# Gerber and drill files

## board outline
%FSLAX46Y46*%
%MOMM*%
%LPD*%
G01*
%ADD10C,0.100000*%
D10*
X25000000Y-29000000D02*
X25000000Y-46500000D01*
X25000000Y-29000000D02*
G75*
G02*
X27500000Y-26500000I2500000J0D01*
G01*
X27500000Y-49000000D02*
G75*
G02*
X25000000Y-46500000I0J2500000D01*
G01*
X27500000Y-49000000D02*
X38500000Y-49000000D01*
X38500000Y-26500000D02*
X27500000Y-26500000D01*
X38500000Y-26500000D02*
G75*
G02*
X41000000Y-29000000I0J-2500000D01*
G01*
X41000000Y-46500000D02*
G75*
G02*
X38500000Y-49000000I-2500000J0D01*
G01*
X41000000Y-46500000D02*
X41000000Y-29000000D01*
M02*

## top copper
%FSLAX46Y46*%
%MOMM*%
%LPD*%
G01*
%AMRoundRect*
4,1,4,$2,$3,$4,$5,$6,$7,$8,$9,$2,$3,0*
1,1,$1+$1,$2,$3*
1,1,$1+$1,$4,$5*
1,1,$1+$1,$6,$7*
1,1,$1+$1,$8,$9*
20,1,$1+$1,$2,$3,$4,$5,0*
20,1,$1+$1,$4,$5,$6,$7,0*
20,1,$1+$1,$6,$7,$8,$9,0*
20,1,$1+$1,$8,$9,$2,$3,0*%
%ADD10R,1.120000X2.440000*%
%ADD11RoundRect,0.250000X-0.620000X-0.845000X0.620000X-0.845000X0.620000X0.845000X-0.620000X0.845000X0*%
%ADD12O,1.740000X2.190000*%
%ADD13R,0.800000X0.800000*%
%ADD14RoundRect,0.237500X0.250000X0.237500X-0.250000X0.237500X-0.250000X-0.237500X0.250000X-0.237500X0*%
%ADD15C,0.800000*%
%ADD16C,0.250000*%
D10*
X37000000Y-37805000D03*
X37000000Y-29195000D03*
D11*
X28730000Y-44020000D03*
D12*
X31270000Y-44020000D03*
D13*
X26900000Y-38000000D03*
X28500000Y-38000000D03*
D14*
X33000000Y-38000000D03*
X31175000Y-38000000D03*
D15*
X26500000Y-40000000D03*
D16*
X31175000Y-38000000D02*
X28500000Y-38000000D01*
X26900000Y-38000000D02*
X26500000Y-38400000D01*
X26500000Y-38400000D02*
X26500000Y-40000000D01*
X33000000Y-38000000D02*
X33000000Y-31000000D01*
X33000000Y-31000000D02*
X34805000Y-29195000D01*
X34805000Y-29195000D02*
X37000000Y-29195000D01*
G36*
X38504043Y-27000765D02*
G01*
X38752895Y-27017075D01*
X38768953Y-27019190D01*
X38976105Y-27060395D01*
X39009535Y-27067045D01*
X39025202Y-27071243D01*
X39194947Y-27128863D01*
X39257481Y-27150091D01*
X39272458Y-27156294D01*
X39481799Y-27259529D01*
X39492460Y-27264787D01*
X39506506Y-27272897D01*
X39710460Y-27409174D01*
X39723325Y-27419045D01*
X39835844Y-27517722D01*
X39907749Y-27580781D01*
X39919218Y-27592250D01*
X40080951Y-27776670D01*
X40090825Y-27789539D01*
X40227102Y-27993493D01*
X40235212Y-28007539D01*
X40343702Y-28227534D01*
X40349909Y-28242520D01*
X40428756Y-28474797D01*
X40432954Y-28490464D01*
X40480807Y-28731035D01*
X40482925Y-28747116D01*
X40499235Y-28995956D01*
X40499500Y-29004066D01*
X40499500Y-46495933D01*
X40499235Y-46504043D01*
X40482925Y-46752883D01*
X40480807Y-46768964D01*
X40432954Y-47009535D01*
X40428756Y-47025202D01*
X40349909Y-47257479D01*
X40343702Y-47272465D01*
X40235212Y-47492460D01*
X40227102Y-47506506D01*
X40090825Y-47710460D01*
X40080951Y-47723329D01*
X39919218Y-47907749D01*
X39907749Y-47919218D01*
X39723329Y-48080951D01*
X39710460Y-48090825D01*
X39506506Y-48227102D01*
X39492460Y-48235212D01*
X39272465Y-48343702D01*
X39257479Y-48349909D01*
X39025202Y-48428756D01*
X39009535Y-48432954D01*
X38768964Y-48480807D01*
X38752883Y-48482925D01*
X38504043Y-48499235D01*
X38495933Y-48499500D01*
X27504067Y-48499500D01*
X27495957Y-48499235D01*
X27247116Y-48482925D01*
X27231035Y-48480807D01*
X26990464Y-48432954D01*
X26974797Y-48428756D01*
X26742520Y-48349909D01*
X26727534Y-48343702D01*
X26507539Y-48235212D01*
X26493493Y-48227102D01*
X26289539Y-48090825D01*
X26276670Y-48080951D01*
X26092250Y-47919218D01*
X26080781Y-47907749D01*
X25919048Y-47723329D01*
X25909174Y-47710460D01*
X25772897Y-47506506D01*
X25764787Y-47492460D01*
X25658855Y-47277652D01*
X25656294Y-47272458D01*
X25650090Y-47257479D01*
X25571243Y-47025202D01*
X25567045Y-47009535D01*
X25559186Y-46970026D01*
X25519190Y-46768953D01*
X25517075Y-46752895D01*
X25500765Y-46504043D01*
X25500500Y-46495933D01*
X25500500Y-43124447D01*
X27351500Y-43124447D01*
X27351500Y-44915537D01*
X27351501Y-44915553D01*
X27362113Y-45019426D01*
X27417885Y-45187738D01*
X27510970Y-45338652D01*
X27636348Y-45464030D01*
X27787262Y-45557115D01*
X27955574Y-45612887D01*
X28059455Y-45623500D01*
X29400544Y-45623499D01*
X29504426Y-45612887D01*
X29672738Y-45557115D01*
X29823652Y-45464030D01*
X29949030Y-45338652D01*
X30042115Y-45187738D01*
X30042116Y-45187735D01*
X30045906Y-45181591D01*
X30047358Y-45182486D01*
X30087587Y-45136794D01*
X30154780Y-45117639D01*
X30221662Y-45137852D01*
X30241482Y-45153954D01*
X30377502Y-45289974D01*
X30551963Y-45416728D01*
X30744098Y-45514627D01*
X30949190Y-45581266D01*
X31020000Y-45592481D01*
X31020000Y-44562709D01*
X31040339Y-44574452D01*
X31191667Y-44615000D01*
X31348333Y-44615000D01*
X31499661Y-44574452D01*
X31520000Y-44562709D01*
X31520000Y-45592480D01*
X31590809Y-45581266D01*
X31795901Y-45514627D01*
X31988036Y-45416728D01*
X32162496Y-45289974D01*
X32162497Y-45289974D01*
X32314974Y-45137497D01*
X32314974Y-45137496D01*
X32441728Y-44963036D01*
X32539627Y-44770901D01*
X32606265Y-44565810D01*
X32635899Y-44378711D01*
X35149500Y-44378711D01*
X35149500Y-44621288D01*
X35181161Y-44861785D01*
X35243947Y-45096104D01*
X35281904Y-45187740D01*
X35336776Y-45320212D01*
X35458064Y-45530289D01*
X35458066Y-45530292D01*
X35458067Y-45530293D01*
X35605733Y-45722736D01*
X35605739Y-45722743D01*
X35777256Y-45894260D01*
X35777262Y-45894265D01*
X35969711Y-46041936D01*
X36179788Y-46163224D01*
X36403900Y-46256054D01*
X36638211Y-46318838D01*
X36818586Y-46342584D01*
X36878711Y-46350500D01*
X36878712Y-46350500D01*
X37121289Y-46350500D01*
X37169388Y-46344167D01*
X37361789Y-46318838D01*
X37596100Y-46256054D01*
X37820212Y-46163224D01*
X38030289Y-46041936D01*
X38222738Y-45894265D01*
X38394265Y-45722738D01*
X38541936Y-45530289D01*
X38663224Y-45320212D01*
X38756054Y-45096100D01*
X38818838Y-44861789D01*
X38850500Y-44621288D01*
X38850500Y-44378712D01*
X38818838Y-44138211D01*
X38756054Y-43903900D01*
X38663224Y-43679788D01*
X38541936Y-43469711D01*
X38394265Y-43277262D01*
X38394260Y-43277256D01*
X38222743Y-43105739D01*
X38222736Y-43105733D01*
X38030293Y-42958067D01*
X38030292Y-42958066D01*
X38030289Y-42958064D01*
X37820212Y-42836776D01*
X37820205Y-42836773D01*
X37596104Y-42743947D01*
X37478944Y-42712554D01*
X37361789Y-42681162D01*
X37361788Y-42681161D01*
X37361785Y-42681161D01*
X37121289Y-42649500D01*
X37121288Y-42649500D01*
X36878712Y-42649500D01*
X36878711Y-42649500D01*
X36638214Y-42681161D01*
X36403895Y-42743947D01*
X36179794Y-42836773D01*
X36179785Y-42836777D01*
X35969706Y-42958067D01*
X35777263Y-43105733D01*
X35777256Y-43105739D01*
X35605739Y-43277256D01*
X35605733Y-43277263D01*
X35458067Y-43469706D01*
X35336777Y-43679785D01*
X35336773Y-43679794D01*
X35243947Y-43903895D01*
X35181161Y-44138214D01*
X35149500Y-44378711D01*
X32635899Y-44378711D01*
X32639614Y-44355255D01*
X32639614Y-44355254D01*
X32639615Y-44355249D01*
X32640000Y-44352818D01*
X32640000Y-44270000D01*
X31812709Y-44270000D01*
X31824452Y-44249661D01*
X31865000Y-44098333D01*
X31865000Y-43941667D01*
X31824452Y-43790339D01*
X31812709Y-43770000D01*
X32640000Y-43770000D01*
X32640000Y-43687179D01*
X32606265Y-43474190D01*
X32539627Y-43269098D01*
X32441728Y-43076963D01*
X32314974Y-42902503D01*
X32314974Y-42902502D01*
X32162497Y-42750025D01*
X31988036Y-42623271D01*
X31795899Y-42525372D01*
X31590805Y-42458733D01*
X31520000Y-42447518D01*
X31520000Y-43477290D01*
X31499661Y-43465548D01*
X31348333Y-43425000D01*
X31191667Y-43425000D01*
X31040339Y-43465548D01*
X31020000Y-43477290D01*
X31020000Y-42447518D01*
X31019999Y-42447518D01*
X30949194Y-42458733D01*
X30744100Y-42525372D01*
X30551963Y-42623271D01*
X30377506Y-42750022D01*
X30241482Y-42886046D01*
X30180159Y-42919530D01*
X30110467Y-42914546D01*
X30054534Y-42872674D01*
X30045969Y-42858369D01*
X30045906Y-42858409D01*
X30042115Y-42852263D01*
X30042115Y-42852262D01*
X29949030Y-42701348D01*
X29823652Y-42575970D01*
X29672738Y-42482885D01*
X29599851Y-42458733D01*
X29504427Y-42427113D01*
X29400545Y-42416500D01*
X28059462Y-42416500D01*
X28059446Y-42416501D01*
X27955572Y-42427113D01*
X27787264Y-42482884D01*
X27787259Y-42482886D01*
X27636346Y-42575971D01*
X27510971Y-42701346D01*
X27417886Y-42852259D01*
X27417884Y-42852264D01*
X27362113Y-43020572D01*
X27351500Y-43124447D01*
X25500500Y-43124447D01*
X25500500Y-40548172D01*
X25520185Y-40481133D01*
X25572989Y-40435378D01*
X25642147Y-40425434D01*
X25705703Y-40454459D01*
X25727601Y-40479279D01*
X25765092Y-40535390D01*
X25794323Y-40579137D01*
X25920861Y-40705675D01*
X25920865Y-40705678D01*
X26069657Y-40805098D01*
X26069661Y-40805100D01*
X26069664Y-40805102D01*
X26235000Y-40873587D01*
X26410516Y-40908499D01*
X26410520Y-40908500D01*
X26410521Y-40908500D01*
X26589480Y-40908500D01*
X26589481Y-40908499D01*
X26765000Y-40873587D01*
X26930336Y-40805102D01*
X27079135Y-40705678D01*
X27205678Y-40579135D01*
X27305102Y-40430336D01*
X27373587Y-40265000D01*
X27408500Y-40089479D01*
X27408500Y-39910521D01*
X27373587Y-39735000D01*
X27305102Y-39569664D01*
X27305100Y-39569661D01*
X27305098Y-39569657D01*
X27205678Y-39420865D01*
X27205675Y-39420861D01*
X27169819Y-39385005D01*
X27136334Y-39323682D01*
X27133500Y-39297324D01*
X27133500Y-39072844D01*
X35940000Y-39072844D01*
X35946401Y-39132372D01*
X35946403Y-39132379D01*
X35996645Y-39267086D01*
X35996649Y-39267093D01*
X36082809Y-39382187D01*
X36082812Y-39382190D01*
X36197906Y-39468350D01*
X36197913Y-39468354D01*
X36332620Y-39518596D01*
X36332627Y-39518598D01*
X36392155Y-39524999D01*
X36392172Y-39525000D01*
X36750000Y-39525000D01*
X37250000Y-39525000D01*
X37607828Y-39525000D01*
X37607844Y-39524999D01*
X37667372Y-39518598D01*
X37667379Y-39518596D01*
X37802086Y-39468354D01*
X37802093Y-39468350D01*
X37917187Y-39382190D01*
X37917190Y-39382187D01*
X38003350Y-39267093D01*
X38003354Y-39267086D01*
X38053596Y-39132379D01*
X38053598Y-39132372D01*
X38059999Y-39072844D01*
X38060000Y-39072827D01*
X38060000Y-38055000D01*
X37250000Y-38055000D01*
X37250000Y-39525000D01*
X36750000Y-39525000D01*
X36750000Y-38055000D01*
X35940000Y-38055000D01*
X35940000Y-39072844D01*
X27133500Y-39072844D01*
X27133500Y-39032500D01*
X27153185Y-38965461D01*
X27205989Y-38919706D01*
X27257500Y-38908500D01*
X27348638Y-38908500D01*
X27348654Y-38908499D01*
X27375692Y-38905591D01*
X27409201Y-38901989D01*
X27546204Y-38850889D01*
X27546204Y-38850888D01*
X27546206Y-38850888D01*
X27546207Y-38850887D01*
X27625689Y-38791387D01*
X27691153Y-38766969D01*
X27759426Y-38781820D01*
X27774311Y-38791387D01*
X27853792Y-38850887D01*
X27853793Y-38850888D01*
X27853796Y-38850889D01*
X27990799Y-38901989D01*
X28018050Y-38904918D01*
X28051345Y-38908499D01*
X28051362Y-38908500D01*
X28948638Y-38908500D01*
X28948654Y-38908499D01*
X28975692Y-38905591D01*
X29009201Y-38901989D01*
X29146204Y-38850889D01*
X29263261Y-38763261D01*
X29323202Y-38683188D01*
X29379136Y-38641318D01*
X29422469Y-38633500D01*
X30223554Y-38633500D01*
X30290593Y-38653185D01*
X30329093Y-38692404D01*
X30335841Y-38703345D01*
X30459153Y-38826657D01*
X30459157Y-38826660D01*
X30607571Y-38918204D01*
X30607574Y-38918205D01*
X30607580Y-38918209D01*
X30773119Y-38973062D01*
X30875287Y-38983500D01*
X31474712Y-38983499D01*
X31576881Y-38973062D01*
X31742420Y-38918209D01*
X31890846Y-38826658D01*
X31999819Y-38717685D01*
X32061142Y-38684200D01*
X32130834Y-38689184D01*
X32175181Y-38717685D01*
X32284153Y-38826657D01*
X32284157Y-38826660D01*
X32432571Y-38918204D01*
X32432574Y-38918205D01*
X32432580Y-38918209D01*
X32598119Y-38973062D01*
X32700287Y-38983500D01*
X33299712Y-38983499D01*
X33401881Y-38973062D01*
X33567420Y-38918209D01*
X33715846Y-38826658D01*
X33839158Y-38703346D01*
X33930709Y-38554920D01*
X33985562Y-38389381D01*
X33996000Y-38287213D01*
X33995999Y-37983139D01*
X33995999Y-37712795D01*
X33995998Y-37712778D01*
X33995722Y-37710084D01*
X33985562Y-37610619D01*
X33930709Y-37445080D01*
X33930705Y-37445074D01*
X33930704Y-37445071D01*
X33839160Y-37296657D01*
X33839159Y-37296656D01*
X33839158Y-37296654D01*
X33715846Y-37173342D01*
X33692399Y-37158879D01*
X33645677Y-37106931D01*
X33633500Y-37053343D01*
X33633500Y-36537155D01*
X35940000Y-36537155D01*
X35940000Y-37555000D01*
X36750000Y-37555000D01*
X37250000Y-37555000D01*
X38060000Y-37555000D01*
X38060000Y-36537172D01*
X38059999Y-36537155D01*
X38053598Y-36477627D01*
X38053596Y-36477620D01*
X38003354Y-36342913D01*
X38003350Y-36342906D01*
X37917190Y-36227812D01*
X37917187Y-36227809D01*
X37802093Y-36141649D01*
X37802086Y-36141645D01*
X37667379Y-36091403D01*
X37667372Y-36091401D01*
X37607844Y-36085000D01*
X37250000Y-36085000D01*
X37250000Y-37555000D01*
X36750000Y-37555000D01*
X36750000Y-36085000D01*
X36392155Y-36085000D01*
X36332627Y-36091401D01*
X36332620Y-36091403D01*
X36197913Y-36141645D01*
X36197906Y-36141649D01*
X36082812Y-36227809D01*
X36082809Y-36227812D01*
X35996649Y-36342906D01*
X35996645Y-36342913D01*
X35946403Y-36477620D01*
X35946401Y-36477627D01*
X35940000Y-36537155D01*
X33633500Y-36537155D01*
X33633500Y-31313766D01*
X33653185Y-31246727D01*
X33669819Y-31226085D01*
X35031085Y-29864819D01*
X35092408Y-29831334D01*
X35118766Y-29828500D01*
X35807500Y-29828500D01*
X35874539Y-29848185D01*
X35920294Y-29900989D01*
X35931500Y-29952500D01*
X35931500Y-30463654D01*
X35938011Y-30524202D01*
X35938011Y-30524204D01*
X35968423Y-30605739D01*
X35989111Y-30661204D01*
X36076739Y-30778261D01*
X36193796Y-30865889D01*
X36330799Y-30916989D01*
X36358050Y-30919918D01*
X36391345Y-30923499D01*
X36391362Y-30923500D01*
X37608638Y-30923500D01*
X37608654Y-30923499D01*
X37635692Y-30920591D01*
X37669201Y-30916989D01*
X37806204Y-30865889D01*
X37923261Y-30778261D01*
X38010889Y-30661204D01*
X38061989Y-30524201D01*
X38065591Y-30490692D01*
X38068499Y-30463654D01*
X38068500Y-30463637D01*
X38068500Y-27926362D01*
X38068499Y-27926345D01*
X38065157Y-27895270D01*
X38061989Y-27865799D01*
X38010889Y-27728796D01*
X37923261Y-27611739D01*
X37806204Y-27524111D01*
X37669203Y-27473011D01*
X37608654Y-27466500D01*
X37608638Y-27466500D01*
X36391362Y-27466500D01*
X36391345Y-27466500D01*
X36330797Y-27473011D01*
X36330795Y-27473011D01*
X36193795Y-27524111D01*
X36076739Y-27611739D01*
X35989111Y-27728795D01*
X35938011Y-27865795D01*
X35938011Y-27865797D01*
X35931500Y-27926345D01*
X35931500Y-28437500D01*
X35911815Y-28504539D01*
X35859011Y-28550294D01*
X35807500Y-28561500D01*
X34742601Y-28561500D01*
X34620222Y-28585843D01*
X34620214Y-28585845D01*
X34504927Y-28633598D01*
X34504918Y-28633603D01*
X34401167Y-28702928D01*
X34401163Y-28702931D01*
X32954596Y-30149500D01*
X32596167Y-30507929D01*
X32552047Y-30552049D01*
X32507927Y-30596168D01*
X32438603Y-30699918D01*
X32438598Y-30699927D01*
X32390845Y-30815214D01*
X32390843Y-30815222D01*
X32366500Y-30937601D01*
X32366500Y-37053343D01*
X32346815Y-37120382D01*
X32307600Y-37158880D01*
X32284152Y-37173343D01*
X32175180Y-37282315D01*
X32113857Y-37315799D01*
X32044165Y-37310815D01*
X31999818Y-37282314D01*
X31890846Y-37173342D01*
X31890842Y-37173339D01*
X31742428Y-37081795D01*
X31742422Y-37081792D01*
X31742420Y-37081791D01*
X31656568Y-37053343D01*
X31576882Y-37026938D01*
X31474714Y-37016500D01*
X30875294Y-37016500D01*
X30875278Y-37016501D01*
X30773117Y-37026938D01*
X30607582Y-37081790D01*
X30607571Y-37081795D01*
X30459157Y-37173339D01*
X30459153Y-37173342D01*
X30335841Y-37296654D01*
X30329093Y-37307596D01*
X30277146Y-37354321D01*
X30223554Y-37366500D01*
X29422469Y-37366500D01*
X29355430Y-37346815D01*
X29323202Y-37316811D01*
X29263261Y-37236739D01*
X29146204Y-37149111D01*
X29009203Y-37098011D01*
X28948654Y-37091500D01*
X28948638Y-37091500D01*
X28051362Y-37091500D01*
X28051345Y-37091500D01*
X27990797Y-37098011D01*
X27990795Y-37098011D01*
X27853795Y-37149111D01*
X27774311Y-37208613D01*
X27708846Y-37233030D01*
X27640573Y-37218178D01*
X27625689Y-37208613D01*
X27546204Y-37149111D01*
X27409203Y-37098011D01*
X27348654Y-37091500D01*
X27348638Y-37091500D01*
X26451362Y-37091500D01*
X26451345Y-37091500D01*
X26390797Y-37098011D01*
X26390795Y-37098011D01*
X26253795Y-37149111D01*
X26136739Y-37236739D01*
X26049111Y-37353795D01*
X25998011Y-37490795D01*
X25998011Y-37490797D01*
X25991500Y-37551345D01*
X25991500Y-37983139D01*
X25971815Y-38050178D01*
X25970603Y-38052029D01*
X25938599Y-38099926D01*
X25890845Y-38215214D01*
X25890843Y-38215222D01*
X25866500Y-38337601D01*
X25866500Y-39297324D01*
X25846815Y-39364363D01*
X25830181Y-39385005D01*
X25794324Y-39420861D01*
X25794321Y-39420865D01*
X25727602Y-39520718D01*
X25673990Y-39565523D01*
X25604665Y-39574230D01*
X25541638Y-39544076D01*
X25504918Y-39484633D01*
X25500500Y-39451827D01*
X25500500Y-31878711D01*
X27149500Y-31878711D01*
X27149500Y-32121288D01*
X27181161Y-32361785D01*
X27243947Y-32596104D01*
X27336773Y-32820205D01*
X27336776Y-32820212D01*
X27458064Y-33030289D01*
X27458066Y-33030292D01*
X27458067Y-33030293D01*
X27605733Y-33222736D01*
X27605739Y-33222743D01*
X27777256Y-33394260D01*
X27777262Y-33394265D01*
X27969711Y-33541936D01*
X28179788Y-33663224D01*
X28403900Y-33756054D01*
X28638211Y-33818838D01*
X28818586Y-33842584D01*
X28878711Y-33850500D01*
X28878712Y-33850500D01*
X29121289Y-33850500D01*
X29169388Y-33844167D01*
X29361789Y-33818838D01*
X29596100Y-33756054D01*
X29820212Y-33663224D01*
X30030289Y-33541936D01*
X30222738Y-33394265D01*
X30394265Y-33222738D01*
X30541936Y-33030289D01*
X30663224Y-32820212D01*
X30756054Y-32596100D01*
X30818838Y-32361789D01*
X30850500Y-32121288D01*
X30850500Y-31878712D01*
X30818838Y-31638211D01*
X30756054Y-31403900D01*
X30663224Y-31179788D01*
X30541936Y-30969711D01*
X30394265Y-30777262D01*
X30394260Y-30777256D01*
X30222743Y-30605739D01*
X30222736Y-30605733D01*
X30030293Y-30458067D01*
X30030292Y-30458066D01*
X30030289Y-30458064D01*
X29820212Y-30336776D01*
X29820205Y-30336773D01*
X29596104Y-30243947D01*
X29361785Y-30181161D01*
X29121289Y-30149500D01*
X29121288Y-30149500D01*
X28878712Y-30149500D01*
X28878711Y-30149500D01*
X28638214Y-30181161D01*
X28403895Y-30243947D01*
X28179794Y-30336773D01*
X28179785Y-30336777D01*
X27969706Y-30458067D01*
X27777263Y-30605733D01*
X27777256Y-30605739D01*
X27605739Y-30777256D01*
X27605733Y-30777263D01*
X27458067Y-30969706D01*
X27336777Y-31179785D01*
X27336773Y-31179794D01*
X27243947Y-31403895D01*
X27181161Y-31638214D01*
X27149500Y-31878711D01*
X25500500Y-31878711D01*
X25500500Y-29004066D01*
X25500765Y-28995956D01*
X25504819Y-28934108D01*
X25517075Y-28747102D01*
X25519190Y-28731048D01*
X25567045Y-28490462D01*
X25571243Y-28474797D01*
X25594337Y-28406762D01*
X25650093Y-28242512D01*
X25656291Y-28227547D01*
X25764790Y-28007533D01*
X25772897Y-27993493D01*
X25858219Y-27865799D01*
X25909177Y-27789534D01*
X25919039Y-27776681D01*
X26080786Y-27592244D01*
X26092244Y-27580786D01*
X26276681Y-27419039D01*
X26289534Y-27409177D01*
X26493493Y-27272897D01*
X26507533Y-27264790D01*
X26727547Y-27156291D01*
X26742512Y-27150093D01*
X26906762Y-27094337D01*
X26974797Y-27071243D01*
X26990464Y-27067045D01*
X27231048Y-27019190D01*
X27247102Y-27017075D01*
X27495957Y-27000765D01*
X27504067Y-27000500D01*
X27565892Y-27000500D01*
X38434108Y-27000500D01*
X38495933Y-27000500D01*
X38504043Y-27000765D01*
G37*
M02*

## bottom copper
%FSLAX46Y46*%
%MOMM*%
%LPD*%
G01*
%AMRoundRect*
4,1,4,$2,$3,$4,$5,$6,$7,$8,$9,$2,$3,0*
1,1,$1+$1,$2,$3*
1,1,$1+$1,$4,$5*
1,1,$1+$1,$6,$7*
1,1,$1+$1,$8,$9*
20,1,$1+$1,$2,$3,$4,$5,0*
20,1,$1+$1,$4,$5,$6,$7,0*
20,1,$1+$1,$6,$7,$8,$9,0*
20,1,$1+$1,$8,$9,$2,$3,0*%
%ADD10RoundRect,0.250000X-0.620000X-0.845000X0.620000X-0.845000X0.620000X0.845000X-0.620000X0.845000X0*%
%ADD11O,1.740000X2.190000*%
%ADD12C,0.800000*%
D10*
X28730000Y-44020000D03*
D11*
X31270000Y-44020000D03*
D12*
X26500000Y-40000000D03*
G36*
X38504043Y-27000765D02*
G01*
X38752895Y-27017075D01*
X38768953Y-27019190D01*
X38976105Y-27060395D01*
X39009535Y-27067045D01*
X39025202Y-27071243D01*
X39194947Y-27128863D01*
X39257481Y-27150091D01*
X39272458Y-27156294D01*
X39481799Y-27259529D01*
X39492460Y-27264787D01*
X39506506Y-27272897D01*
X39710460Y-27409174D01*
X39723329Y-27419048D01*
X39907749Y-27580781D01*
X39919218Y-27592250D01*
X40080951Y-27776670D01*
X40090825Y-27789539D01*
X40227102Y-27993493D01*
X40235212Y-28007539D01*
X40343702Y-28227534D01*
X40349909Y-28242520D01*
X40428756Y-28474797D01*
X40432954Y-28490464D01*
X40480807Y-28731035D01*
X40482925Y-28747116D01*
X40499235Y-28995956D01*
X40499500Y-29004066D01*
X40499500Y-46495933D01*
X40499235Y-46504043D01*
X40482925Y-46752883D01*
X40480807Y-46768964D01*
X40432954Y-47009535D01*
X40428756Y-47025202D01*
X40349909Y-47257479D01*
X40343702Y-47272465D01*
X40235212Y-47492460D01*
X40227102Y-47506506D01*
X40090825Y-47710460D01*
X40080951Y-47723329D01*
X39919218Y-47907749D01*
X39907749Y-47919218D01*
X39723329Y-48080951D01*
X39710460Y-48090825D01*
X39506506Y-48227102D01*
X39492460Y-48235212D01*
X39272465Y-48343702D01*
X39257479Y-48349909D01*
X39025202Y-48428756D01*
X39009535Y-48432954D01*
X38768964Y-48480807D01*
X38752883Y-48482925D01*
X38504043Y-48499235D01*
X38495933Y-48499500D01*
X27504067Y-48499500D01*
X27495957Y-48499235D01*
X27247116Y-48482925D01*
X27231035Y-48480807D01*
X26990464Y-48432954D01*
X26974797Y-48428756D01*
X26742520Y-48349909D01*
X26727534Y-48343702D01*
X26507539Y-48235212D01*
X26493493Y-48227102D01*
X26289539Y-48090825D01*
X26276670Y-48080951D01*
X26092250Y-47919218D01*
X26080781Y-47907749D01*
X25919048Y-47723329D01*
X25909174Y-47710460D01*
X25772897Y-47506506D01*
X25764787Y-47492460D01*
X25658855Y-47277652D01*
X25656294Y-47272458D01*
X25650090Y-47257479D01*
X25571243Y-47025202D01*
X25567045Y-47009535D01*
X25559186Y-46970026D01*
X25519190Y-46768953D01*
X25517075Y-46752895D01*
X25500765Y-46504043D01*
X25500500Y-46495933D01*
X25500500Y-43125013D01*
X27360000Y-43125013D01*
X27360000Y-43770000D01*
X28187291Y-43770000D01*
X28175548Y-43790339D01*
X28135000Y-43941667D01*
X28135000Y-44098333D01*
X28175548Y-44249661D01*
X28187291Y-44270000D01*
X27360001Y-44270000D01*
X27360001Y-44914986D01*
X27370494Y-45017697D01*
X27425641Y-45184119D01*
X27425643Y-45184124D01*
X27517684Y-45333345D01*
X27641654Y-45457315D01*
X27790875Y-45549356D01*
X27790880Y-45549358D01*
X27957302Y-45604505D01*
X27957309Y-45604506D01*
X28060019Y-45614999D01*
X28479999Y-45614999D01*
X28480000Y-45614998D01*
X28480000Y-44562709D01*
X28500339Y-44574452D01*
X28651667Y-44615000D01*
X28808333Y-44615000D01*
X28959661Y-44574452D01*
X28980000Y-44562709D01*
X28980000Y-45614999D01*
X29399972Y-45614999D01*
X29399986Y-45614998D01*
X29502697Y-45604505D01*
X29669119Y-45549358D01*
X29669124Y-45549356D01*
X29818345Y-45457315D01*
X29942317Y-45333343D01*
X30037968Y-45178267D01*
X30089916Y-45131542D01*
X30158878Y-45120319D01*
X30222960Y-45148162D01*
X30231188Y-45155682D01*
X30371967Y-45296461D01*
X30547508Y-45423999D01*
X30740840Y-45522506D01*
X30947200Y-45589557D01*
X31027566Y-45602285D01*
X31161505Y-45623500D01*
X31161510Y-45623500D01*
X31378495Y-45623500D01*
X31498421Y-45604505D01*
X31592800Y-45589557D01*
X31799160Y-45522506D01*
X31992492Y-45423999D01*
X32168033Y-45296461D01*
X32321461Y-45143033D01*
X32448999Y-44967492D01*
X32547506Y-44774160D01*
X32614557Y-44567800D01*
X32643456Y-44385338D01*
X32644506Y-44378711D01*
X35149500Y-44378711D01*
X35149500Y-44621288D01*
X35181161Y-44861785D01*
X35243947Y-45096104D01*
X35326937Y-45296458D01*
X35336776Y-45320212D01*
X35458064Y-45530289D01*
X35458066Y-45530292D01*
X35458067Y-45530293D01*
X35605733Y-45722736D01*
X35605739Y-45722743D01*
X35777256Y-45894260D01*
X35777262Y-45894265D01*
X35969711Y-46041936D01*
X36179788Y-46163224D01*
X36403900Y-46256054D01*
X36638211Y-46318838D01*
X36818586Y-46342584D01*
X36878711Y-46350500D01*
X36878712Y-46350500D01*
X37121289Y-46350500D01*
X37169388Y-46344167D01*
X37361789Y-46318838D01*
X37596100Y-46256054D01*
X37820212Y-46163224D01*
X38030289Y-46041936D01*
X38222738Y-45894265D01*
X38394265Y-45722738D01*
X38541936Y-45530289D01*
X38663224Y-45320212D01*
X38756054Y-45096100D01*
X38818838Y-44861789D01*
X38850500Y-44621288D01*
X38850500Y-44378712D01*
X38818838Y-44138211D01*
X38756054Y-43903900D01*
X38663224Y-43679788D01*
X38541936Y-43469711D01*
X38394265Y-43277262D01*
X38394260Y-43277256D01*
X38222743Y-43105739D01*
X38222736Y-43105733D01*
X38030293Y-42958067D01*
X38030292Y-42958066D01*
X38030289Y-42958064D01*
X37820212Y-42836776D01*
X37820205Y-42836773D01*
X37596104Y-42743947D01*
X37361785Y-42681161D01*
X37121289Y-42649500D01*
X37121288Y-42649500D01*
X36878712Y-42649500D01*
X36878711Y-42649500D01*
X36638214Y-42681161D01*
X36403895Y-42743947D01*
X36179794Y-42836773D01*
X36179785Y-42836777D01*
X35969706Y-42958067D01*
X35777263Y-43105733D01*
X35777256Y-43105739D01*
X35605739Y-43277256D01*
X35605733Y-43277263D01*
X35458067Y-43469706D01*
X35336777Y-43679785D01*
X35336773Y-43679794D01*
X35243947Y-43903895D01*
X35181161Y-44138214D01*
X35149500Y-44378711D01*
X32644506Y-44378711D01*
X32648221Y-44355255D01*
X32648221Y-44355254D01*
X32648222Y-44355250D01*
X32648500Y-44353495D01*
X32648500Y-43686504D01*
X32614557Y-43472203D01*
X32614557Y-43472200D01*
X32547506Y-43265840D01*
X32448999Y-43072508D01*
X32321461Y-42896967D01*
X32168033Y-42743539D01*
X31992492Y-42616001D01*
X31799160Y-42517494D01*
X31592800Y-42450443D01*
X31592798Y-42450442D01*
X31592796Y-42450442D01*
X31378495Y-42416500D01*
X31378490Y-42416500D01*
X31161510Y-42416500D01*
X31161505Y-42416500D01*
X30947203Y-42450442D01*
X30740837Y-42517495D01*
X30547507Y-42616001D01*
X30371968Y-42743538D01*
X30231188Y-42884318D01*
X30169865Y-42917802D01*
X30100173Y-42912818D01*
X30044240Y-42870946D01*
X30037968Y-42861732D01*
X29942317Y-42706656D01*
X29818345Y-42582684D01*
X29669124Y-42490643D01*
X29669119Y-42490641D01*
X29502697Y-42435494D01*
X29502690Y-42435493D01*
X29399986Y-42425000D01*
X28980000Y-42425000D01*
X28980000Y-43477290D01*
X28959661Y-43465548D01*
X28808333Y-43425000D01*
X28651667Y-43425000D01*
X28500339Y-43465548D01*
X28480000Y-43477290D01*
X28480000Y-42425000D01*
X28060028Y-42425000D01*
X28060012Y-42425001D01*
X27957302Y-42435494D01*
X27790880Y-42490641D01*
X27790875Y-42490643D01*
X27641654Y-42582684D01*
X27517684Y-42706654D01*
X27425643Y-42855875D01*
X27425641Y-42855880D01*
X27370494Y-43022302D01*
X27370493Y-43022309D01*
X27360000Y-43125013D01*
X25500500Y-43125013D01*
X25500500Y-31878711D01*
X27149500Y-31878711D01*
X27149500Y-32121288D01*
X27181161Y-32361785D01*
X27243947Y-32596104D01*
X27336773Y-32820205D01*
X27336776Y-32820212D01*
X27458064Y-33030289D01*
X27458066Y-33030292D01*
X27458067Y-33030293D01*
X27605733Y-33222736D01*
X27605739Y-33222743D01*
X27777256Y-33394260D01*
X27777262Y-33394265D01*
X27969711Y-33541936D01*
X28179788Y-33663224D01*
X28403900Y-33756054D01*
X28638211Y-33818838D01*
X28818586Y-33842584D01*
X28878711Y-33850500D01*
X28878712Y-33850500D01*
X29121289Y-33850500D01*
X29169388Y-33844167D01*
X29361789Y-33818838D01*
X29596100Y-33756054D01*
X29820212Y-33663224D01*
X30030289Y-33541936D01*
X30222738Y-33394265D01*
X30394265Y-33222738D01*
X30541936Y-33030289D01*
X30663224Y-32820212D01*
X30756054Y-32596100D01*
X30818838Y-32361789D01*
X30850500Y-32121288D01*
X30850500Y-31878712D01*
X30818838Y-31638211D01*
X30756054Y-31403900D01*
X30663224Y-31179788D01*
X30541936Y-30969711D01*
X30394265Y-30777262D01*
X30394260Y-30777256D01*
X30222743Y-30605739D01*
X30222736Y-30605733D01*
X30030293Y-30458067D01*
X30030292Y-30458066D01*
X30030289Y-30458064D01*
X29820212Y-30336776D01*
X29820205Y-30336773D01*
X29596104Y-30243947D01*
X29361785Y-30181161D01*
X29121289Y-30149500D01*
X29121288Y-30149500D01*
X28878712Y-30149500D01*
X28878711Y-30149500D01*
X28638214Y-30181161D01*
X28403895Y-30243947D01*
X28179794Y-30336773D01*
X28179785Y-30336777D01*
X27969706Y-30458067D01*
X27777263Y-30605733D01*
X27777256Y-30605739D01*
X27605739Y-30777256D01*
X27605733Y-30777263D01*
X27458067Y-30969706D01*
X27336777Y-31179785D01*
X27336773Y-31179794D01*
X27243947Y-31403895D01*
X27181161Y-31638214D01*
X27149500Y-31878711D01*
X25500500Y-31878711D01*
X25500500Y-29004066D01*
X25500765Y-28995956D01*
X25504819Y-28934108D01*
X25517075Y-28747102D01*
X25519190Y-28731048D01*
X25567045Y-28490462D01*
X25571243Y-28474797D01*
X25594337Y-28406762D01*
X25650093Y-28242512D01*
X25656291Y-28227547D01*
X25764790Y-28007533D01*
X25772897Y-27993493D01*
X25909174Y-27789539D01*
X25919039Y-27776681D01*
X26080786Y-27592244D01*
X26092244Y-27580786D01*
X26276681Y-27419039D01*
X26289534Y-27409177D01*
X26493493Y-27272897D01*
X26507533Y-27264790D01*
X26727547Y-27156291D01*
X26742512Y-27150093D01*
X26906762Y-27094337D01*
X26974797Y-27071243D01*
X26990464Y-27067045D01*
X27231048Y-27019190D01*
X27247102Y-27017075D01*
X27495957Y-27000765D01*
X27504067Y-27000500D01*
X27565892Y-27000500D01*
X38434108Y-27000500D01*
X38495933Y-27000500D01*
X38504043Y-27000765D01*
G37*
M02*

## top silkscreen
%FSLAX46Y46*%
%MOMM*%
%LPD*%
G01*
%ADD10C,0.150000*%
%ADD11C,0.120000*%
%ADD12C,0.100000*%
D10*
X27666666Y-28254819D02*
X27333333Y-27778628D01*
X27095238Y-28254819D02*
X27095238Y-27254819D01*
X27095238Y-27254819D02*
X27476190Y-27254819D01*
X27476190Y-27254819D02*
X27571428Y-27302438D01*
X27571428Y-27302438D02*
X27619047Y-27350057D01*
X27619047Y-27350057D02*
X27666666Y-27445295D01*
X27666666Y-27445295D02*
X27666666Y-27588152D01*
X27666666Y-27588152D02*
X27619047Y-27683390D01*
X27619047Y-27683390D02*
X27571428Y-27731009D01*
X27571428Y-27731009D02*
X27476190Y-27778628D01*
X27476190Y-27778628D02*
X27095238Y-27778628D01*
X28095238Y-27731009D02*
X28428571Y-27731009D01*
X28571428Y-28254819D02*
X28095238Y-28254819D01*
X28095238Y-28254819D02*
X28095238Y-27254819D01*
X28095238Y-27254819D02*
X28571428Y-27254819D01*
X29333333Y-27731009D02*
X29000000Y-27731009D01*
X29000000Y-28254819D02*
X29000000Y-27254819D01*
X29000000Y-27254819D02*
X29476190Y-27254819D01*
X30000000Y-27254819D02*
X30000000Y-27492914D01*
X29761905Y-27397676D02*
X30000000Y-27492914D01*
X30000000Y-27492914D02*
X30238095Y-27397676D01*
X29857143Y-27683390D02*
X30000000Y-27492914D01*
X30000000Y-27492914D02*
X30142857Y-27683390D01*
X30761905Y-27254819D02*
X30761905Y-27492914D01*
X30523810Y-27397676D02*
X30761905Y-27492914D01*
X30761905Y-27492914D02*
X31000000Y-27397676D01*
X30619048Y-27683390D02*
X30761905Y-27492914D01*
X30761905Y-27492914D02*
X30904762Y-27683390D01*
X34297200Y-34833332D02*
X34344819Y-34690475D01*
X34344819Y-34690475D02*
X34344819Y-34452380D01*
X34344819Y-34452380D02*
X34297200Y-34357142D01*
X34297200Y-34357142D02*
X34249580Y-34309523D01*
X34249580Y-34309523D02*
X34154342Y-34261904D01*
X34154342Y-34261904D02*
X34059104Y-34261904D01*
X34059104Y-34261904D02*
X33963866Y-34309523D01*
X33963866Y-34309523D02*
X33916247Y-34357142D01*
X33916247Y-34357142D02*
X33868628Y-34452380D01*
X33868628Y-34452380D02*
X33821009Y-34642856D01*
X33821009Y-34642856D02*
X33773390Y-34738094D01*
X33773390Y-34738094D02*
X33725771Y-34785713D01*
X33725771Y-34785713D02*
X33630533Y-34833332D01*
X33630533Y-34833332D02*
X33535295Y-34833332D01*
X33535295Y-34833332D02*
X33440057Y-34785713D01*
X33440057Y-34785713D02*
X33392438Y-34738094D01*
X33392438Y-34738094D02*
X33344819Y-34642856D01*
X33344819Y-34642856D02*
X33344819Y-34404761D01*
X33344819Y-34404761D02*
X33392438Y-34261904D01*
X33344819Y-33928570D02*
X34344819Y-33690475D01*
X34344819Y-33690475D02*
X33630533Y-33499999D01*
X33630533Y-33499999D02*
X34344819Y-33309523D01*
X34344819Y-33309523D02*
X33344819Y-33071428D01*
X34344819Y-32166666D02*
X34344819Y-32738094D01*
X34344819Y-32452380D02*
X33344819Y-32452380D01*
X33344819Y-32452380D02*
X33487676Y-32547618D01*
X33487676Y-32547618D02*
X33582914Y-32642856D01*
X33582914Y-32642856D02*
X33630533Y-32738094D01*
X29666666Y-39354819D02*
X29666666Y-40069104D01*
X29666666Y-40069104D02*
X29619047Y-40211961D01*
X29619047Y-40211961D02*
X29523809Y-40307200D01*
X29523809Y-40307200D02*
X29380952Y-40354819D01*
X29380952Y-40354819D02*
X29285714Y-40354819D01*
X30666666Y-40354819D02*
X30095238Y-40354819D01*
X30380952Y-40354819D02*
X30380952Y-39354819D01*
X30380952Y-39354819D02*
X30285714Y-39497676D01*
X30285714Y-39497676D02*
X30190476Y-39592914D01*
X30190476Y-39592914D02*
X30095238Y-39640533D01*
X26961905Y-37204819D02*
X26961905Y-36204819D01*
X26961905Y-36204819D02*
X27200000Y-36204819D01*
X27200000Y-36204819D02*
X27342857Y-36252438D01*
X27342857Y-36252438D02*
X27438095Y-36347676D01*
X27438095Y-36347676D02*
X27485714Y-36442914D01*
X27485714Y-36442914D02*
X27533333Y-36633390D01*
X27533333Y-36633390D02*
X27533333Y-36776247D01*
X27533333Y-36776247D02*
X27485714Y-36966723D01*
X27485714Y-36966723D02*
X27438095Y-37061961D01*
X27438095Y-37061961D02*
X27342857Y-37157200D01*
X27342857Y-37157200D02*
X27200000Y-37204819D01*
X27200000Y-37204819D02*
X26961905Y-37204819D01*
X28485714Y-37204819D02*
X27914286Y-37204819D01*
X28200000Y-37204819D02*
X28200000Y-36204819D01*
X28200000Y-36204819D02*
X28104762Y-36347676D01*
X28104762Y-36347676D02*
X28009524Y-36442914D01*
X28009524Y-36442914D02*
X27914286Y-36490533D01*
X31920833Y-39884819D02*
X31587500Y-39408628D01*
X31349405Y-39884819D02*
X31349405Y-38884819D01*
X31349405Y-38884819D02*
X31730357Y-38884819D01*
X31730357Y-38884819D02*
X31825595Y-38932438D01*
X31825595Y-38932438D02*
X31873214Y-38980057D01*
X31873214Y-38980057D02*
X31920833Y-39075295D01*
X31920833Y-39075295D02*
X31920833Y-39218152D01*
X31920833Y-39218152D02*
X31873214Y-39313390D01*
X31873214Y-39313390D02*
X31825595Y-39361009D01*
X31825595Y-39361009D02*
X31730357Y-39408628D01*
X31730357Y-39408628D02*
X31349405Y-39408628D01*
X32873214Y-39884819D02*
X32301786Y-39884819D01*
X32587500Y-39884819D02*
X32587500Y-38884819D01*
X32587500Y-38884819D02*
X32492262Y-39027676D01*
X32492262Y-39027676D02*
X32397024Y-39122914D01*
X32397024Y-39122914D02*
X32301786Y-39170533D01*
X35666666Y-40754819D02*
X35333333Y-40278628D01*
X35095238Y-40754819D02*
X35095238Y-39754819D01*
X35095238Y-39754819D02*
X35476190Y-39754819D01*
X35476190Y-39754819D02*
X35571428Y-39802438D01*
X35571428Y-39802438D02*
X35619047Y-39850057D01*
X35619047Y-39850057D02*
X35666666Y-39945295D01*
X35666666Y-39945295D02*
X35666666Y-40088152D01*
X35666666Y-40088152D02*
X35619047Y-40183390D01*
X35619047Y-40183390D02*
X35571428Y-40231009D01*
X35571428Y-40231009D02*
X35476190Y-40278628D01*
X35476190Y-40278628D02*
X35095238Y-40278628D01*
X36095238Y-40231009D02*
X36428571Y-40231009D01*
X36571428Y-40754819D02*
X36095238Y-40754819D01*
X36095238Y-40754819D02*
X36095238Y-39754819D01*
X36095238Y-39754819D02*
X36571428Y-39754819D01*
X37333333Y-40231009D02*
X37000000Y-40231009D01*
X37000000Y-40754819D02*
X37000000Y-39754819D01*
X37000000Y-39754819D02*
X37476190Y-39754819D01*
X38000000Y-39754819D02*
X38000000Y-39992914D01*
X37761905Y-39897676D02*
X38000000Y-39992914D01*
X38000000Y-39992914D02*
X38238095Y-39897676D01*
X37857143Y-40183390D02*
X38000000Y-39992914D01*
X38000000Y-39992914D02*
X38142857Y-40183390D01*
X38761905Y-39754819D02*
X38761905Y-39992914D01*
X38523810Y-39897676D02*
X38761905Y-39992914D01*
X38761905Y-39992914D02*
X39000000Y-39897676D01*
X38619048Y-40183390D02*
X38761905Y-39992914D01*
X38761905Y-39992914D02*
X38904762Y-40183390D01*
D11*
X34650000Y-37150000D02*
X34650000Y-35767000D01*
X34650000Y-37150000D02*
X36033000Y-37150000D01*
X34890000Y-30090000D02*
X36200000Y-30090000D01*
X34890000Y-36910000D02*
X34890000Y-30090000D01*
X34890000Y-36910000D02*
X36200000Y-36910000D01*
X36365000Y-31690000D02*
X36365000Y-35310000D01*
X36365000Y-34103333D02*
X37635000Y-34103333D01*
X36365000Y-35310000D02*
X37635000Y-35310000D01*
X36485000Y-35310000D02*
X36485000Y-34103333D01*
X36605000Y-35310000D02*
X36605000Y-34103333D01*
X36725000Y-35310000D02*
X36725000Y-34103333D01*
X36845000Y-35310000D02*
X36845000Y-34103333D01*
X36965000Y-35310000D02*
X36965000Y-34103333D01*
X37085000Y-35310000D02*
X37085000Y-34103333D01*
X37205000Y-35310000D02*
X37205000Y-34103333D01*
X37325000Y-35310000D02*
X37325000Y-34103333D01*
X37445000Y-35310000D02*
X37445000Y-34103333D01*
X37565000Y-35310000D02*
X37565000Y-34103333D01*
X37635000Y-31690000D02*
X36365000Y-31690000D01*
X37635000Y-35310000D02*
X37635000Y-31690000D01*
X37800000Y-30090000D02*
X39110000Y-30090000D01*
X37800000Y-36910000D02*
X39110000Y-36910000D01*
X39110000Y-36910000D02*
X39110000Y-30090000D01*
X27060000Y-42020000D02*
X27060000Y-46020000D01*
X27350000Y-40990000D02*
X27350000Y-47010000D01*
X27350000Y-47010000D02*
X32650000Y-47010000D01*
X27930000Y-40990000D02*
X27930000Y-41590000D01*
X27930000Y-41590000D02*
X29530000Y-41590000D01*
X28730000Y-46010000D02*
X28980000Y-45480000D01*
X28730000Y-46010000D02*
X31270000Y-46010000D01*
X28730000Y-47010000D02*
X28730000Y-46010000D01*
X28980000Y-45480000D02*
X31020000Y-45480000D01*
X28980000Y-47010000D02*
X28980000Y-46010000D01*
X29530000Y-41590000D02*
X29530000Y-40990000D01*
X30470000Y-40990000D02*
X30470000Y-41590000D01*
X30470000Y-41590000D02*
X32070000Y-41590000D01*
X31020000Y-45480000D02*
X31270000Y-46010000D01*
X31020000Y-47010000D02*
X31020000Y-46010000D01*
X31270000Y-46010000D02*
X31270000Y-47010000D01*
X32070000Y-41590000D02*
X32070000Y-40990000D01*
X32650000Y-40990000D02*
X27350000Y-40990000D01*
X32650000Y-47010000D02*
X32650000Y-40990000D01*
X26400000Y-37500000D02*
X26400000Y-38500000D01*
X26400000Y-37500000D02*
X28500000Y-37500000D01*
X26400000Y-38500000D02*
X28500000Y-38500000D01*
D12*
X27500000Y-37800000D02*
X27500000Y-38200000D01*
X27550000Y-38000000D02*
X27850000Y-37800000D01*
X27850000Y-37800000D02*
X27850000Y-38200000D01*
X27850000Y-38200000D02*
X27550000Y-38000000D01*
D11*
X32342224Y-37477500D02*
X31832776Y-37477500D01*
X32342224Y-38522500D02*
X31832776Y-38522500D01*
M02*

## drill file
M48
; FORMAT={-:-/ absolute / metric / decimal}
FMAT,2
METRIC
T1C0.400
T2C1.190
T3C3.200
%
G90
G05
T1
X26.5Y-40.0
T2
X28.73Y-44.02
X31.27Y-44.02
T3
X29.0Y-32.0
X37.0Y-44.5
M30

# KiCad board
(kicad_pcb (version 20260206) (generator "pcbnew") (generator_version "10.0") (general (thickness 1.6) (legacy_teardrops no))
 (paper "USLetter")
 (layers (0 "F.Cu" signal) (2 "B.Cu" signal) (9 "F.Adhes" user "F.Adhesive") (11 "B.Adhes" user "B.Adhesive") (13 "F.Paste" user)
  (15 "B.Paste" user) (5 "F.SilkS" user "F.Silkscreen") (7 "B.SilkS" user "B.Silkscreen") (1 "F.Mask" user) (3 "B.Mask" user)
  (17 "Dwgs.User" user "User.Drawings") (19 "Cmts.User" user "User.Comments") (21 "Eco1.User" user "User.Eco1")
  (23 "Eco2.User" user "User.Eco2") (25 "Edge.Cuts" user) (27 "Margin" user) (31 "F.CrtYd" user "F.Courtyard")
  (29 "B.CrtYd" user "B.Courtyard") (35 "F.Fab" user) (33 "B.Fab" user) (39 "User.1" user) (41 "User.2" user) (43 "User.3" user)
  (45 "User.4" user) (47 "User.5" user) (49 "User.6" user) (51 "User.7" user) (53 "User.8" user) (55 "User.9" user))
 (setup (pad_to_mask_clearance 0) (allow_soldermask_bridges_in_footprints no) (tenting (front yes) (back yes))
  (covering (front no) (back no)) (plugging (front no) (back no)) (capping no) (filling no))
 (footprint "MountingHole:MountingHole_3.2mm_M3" (layer "F.Cu") (at 29 32)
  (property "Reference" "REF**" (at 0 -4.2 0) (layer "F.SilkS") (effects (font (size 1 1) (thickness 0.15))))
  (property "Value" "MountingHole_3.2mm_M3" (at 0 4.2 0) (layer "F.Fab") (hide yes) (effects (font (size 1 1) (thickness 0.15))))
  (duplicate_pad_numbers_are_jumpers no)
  (pad "" np_thru_hole circle (at 0 0) (size 3.2 3.2) (drill 3.2) (layers "*.Cu" "*.Mask")))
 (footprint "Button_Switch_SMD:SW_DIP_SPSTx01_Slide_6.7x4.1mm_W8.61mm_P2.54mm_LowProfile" (layer "F.Cu") (at 37 33.5 90)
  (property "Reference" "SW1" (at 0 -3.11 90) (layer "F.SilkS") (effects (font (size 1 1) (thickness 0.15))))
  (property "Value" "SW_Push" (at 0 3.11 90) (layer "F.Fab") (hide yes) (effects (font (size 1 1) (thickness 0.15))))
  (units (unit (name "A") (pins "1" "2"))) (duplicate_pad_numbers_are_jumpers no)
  (fp_line (start -3.65 -2.35) (end -2.267 -2.35) (stroke (width 0.12) (type solid)) (layer "F.SilkS"))
  (fp_line (start -3.65 -2.35) (end -3.65 -0.967) (stroke (width 0.12) (type solid)) (layer "F.SilkS"))
  (fp_line (start 3.41 -2.11) (end 3.41 -0.8) (stroke (width 0.12) (type solid)) (layer "F.SilkS"))
  (fp_line (start -3.41 -2.11) (end 3.41 -2.11) (stroke (width 0.12) (type solid)) (layer "F.SilkS"))
  (fp_line (start -3.41 -2.11) (end -3.41 -0.8) (stroke (width 0.12) (type solid)) (layer "F.SilkS"))
  (fp_line (start 1.81 -0.635) (end -1.81 -0.635) (stroke (width 0.12) (type solid)) (layer "F.SilkS"))
  (fp_line (start -0.603333 -0.635) (end -0.603333 0.635) (stroke (width 0.12) (type solid)) (layer "F.SilkS"))
  (fp_line (start -1.81 -0.635) (end -1.81 0.635) (stroke (width 0.12) (type solid)) (layer "F.SilkS"))
  (fp_line (start -1.81 -0.515) (end -0.603333 -0.515) (stroke (width 0.12) (type solid)) (layer "F.SilkS"))
  (fp_line (start -1.81 -0.395) (end -0.603333 -0.395) (stroke (width 0.12) (type solid)) (layer "F.SilkS"))
  (fp_line (start -1.81 -0.275) (end -0.603333 -0.275) (stroke (width 0.12) (type solid)) (layer "F.SilkS"))
  (fp_line (start -1.81 -0.155) (end -0.603333 -0.155) (stroke (width 0.12) (type solid)) (layer "F.SilkS"))
  (fp_line (start -1.81 -0.035) (end -0.603333 -0.035) (stroke (width 0.12) (type solid)) (layer "F.SilkS"))
  (fp_line (start -1.81 0.085) (end -0.603333 0.085) (stroke (width 0.12) (type solid)) (layer "F.SilkS"))
  (fp_line (start -1.81 0.205) (end -0.603333 0.205) (stroke (width 0.12) (type solid)) (layer "F.SilkS"))
  (fp_line (start -1.81 0.325) (end -0.603333 0.325) (stroke (width 0.12) (type solid)) (layer "F.SilkS"))
  (fp_line (start -1.81 0.445) (end -0.603333 0.445) (stroke (width 0.12) (type solid)) (layer "F.SilkS"))
  (fp_line (start -1.81 0.565) (end -0.603333 0.565) (stroke (width 0.12) (type solid)) (layer "F.SilkS"))
  (fp_line (start 1.81 0.635) (end 1.81 -0.635) (stroke (width 0.12) (type solid)) (layer "F.SilkS"))
  (fp_line (start -1.81 0.635) (end 1.81 0.635) (stroke (width 0.12) (type solid)) (layer "F.SilkS"))
  (fp_line (start 3.41 0.8) (end 3.41 2.11) (stroke (width 0.12) (type solid)) (layer "F.SilkS"))
  (fp_line (start -3.41 0.8) (end -3.41 2.11) (stroke (width 0.12) (type solid)) (layer "F.SilkS"))
  (fp_line (start -3.41 2.11) (end 3.41 2.11) (stroke (width 0.12) (type solid)) (layer "F.SilkS"))
  (pad "1" smd rect (at -4.305 0 90) (size 2.44 1.12) (layers "F.Cu" "F.Mask" "F.Paste") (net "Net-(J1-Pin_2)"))
  (pad "2" smd rect (at 4.305 0 90) (size 2.44 1.12) (layers "F.Cu" "F.Mask" "F.Paste") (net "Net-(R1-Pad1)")))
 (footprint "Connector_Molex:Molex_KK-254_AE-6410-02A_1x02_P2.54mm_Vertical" (layer "F.Cu") (at 28.73 44.02)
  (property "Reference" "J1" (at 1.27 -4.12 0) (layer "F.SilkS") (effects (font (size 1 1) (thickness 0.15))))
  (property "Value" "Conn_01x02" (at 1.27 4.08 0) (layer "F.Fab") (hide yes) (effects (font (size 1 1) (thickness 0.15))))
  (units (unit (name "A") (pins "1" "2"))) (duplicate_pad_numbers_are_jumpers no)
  (fp_line (start -1.67 -2) (end -1.67 2) (stroke (width 0.12) (type solid)) (layer "F.SilkS"))
  (fp_line (start -1.38 -3.03) (end -1.38 2.99) (stroke (width 0.12) (type solid)) (layer "F.SilkS"))
  (fp_line (start -1.38 2.99) (end 3.92 2.99) (stroke (width 0.12) (type solid)) (layer "F.SilkS"))
  (fp_line (start -0.8 -3.03) (end -0.8 -2.43) (stroke (width 0.12) (type solid)) (layer "F.SilkS"))
  (fp_line (start -0.8 -2.43) (end 0.8 -2.43) (stroke (width 0.12) (type solid)) (layer "F.SilkS"))
  (fp_line (start 0 1.99) (end 0.25 1.46) (stroke (width 0.12) (type solid)) (layer "F.SilkS"))
  (fp_line (start 0 1.99) (end 2.54 1.99) (stroke (width 0.12) (type solid)) (layer "F.SilkS"))
  (fp_line (start 0 2.99) (end 0 1.99) (stroke (width 0.12) (type solid)) (layer "F.SilkS"))
  (fp_line (start 0.25 1.46) (end 2.29 1.46) (stroke (width 0.12) (type solid)) (layer "F.SilkS"))
  (fp_line (start 0.25 2.99) (end 0.25 1.99) (stroke (width 0.12) (type solid)) (layer "F.SilkS"))
  (fp_line (start 0.8 -2.43) (end 0.8 -3.03) (stroke (width 0.12) (type solid)) (layer "F.SilkS"))
  (fp_line (start 1.74 -3.03) (end 1.74 -2.43) (stroke (width 0.12) (type solid)) (layer "F.SilkS"))
  (fp_line (start 1.74 -2.43) (end 3.34 -2.43) (stroke (width 0.12) (type solid)) (layer "F.SilkS"))
  (fp_line (start 2.29 1.46) (end 2.54 1.99) (stroke (width 0.12) (type solid)) (layer "F.SilkS"))
  (fp_line (start 2.29 2.99) (end 2.29 1.99) (stroke (width 0.12) (type solid)) (layer "F.SilkS"))
  (fp_line (start 2.54 1.99) (end 2.54 2.99) (stroke (width 0.12) (type solid)) (layer "F.SilkS"))
  (fp_line (start 3.34 -2.43) (end 3.34 -3.03) (stroke (width 0.12) (type solid)) (layer "F.SilkS"))
  (fp_line (start 3.92 -3.03) (end -1.38 -3.03) (stroke (width 0.12) (type solid)) (layer "F.SilkS"))
  (fp_line (start 3.92 2.99) (end 3.92 -3.03) (stroke (width 0.12) (type solid)) (layer "F.SilkS"))
  (pad "1" thru_hole roundrect (at 0 0) (size 1.74 2.19) (drill 1.19) (layers "*.Cu" "*.Mask") (remove_unused_layers no)
   (roundrect_rratio 0.143678) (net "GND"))
  (pad "2" thru_hole oval (at 2.54 0) (size 1.74 2.19) (drill 1.19) (layers "*.Cu" "*.Mask") (remove_unused_layers no)
   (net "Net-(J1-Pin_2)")))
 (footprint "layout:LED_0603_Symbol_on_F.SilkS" (layer "F.Cu") (at 27.7 38)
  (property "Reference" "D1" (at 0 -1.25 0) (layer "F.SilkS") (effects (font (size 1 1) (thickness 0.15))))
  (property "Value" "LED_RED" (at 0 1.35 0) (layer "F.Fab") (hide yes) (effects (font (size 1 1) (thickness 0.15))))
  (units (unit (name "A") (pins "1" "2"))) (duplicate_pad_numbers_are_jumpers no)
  (fp_line (start -1.3 -0.5) (end -1.3 0.5) (stroke (width 0.12) (type solid)) (layer "F.SilkS"))
  (fp_line (start -1.3 -0.5) (end 0.8 -0.5) (stroke (width 0.12) (type solid)) (layer "F.SilkS"))
  (fp_line (start -1.3 0.5) (end 0.8 0.5) (stroke (width 0.12) (type solid)) (layer "F.SilkS"))
  (fp_line (start -0.2 -0.2) (end -0.2 0.2) (stroke (width 0.1) (type solid)) (layer "F.SilkS"))
  (fp_line (start -0.15 0) (end 0.15 -0.2) (stroke (width 0.1) (type solid)) (layer "F.SilkS"))
  (fp_line (start 0.15 -0.2) (end 0.15 0.2) (stroke (width 0.1) (type solid)) (layer "F.SilkS"))
  (fp_line (start 0.15 0.2) (end -0.15 0) (stroke (width 0.1) (type solid)) (layer "F.SilkS"))
  (pad "1" smd rect (at -0.8 0 180) (size 0.8 0.8) (layers "F.Cu" "F.Mask" "F.Paste") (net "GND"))
  (pad "2" smd rect (at 0.8 0 180) (size 0.8 0.8) (layers "F.Cu" "F.Mask" "F.Paste") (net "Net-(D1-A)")))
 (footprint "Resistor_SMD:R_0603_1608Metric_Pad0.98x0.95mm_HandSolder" (layer "F.Cu") (at 32.0875 38 180)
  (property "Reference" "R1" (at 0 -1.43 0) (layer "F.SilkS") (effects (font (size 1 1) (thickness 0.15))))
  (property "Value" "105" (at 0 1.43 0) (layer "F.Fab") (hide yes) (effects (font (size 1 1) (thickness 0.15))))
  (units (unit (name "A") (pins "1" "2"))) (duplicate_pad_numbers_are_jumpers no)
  (fp_line (start -0.254724 0.5225) (end 0.254724 0.5225) (stroke (width 0.12) (type solid)) (layer "F.SilkS"))
  (fp_line (start -0.254724 -0.5225) (end 0.254724 -0.5225) (stroke (width 0.12) (type solid)) (layer "F.SilkS"))
  (pad "1" smd roundrect (at -0.9125 0 180) (size 0.975 0.95) (layers "F.Cu" "F.Mask" "F.Paste") (roundrect_rratio 0.25)
   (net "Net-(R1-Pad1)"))
  (pad "2" smd roundrect (at 0.9125 0 180) (size 0.975 0.95) (layers "F.Cu" "F.Mask" "F.Paste") (roundrect_rratio 0.25) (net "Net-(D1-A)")))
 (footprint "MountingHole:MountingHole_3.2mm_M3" (layer "F.Cu") (at 37 44.5)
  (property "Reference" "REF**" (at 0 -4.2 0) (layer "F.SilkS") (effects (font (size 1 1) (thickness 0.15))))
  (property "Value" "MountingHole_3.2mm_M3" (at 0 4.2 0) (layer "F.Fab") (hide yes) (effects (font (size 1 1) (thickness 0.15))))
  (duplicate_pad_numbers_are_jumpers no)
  (pad "" np_thru_hole circle (at 0 0) (size 3.2 3.2) (drill 3.2) (layers "*.Cu" "*.Mask")))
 (gr_line (start 25 29) (end 25 46.5) (stroke (width 0.1) (type default)) (layer "Edge.Cuts"))
 (gr_arc (start 25 29) (mid 25.732233 27.232233) (end 27.5 26.5) (stroke (width 0.1) (type default)) (layer "Edge.Cuts"))
 (gr_arc (start 27.5 49) (mid 25.732233 48.267767) (end 25 46.5) (stroke (width 0.1) (type default)) (layer "Edge.Cuts"))
 (gr_line (start 27.5 49) (end 38.5 49) (stroke (width 0.1) (type default)) (layer "Edge.Cuts"))
 (gr_line (start 38.5 26.5) (end 27.5 26.5) (stroke (width 0.1) (type default)) (layer "Edge.Cuts"))
 (gr_arc (start 38.5 26.5) (mid 40.267767 27.232233) (end 41 29) (stroke (width 0.1) (type default)) (layer "Edge.Cuts"))
 (gr_arc (start 41 46.5) (mid 40.267767 48.267767) (end 38.5 49) (stroke (width 0.1) (type default)) (layer "Edge.Cuts"))
 (gr_line (start 41 46.5) (end 41 29) (stroke (width 0.1) (type default)) (layer "Edge.Cuts"))
 (segment (start 31.175 38) (end 28.5 38) (width 0.25) (layer "F.Cu") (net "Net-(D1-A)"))
 (segment (start 26.9 38) (end 26.5 38.4) (width 0.25) (layer "F.Cu") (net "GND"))
 (segment (start 26.5 38.4) (end 26.5 40) (width 0.25) (layer "F.Cu") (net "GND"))
 (via (at 26.5 40) (size 0.8) (drill 0.4) (layers "F.Cu" "B.Cu") (free yes) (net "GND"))
 (segment (start 33 38) (end 33 31) (width 0.25) (layer "F.Cu") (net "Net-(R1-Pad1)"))
 (segment (start 33 31) (end 34.805 29.195) (width 0.25) (layer "F.Cu") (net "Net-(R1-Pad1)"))
 (segment (start 34.805 29.195) (end 37 29.195) (width 0.25) (layer "F.Cu") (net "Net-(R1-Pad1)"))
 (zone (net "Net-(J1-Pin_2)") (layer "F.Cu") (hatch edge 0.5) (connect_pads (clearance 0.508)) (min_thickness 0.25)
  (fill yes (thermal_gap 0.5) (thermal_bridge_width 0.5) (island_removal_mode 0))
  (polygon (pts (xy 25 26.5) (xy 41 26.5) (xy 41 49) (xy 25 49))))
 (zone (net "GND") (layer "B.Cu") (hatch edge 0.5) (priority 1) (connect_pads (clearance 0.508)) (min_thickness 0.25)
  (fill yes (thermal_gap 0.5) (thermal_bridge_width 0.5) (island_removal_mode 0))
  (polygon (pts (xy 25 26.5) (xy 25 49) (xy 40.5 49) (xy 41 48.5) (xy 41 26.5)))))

